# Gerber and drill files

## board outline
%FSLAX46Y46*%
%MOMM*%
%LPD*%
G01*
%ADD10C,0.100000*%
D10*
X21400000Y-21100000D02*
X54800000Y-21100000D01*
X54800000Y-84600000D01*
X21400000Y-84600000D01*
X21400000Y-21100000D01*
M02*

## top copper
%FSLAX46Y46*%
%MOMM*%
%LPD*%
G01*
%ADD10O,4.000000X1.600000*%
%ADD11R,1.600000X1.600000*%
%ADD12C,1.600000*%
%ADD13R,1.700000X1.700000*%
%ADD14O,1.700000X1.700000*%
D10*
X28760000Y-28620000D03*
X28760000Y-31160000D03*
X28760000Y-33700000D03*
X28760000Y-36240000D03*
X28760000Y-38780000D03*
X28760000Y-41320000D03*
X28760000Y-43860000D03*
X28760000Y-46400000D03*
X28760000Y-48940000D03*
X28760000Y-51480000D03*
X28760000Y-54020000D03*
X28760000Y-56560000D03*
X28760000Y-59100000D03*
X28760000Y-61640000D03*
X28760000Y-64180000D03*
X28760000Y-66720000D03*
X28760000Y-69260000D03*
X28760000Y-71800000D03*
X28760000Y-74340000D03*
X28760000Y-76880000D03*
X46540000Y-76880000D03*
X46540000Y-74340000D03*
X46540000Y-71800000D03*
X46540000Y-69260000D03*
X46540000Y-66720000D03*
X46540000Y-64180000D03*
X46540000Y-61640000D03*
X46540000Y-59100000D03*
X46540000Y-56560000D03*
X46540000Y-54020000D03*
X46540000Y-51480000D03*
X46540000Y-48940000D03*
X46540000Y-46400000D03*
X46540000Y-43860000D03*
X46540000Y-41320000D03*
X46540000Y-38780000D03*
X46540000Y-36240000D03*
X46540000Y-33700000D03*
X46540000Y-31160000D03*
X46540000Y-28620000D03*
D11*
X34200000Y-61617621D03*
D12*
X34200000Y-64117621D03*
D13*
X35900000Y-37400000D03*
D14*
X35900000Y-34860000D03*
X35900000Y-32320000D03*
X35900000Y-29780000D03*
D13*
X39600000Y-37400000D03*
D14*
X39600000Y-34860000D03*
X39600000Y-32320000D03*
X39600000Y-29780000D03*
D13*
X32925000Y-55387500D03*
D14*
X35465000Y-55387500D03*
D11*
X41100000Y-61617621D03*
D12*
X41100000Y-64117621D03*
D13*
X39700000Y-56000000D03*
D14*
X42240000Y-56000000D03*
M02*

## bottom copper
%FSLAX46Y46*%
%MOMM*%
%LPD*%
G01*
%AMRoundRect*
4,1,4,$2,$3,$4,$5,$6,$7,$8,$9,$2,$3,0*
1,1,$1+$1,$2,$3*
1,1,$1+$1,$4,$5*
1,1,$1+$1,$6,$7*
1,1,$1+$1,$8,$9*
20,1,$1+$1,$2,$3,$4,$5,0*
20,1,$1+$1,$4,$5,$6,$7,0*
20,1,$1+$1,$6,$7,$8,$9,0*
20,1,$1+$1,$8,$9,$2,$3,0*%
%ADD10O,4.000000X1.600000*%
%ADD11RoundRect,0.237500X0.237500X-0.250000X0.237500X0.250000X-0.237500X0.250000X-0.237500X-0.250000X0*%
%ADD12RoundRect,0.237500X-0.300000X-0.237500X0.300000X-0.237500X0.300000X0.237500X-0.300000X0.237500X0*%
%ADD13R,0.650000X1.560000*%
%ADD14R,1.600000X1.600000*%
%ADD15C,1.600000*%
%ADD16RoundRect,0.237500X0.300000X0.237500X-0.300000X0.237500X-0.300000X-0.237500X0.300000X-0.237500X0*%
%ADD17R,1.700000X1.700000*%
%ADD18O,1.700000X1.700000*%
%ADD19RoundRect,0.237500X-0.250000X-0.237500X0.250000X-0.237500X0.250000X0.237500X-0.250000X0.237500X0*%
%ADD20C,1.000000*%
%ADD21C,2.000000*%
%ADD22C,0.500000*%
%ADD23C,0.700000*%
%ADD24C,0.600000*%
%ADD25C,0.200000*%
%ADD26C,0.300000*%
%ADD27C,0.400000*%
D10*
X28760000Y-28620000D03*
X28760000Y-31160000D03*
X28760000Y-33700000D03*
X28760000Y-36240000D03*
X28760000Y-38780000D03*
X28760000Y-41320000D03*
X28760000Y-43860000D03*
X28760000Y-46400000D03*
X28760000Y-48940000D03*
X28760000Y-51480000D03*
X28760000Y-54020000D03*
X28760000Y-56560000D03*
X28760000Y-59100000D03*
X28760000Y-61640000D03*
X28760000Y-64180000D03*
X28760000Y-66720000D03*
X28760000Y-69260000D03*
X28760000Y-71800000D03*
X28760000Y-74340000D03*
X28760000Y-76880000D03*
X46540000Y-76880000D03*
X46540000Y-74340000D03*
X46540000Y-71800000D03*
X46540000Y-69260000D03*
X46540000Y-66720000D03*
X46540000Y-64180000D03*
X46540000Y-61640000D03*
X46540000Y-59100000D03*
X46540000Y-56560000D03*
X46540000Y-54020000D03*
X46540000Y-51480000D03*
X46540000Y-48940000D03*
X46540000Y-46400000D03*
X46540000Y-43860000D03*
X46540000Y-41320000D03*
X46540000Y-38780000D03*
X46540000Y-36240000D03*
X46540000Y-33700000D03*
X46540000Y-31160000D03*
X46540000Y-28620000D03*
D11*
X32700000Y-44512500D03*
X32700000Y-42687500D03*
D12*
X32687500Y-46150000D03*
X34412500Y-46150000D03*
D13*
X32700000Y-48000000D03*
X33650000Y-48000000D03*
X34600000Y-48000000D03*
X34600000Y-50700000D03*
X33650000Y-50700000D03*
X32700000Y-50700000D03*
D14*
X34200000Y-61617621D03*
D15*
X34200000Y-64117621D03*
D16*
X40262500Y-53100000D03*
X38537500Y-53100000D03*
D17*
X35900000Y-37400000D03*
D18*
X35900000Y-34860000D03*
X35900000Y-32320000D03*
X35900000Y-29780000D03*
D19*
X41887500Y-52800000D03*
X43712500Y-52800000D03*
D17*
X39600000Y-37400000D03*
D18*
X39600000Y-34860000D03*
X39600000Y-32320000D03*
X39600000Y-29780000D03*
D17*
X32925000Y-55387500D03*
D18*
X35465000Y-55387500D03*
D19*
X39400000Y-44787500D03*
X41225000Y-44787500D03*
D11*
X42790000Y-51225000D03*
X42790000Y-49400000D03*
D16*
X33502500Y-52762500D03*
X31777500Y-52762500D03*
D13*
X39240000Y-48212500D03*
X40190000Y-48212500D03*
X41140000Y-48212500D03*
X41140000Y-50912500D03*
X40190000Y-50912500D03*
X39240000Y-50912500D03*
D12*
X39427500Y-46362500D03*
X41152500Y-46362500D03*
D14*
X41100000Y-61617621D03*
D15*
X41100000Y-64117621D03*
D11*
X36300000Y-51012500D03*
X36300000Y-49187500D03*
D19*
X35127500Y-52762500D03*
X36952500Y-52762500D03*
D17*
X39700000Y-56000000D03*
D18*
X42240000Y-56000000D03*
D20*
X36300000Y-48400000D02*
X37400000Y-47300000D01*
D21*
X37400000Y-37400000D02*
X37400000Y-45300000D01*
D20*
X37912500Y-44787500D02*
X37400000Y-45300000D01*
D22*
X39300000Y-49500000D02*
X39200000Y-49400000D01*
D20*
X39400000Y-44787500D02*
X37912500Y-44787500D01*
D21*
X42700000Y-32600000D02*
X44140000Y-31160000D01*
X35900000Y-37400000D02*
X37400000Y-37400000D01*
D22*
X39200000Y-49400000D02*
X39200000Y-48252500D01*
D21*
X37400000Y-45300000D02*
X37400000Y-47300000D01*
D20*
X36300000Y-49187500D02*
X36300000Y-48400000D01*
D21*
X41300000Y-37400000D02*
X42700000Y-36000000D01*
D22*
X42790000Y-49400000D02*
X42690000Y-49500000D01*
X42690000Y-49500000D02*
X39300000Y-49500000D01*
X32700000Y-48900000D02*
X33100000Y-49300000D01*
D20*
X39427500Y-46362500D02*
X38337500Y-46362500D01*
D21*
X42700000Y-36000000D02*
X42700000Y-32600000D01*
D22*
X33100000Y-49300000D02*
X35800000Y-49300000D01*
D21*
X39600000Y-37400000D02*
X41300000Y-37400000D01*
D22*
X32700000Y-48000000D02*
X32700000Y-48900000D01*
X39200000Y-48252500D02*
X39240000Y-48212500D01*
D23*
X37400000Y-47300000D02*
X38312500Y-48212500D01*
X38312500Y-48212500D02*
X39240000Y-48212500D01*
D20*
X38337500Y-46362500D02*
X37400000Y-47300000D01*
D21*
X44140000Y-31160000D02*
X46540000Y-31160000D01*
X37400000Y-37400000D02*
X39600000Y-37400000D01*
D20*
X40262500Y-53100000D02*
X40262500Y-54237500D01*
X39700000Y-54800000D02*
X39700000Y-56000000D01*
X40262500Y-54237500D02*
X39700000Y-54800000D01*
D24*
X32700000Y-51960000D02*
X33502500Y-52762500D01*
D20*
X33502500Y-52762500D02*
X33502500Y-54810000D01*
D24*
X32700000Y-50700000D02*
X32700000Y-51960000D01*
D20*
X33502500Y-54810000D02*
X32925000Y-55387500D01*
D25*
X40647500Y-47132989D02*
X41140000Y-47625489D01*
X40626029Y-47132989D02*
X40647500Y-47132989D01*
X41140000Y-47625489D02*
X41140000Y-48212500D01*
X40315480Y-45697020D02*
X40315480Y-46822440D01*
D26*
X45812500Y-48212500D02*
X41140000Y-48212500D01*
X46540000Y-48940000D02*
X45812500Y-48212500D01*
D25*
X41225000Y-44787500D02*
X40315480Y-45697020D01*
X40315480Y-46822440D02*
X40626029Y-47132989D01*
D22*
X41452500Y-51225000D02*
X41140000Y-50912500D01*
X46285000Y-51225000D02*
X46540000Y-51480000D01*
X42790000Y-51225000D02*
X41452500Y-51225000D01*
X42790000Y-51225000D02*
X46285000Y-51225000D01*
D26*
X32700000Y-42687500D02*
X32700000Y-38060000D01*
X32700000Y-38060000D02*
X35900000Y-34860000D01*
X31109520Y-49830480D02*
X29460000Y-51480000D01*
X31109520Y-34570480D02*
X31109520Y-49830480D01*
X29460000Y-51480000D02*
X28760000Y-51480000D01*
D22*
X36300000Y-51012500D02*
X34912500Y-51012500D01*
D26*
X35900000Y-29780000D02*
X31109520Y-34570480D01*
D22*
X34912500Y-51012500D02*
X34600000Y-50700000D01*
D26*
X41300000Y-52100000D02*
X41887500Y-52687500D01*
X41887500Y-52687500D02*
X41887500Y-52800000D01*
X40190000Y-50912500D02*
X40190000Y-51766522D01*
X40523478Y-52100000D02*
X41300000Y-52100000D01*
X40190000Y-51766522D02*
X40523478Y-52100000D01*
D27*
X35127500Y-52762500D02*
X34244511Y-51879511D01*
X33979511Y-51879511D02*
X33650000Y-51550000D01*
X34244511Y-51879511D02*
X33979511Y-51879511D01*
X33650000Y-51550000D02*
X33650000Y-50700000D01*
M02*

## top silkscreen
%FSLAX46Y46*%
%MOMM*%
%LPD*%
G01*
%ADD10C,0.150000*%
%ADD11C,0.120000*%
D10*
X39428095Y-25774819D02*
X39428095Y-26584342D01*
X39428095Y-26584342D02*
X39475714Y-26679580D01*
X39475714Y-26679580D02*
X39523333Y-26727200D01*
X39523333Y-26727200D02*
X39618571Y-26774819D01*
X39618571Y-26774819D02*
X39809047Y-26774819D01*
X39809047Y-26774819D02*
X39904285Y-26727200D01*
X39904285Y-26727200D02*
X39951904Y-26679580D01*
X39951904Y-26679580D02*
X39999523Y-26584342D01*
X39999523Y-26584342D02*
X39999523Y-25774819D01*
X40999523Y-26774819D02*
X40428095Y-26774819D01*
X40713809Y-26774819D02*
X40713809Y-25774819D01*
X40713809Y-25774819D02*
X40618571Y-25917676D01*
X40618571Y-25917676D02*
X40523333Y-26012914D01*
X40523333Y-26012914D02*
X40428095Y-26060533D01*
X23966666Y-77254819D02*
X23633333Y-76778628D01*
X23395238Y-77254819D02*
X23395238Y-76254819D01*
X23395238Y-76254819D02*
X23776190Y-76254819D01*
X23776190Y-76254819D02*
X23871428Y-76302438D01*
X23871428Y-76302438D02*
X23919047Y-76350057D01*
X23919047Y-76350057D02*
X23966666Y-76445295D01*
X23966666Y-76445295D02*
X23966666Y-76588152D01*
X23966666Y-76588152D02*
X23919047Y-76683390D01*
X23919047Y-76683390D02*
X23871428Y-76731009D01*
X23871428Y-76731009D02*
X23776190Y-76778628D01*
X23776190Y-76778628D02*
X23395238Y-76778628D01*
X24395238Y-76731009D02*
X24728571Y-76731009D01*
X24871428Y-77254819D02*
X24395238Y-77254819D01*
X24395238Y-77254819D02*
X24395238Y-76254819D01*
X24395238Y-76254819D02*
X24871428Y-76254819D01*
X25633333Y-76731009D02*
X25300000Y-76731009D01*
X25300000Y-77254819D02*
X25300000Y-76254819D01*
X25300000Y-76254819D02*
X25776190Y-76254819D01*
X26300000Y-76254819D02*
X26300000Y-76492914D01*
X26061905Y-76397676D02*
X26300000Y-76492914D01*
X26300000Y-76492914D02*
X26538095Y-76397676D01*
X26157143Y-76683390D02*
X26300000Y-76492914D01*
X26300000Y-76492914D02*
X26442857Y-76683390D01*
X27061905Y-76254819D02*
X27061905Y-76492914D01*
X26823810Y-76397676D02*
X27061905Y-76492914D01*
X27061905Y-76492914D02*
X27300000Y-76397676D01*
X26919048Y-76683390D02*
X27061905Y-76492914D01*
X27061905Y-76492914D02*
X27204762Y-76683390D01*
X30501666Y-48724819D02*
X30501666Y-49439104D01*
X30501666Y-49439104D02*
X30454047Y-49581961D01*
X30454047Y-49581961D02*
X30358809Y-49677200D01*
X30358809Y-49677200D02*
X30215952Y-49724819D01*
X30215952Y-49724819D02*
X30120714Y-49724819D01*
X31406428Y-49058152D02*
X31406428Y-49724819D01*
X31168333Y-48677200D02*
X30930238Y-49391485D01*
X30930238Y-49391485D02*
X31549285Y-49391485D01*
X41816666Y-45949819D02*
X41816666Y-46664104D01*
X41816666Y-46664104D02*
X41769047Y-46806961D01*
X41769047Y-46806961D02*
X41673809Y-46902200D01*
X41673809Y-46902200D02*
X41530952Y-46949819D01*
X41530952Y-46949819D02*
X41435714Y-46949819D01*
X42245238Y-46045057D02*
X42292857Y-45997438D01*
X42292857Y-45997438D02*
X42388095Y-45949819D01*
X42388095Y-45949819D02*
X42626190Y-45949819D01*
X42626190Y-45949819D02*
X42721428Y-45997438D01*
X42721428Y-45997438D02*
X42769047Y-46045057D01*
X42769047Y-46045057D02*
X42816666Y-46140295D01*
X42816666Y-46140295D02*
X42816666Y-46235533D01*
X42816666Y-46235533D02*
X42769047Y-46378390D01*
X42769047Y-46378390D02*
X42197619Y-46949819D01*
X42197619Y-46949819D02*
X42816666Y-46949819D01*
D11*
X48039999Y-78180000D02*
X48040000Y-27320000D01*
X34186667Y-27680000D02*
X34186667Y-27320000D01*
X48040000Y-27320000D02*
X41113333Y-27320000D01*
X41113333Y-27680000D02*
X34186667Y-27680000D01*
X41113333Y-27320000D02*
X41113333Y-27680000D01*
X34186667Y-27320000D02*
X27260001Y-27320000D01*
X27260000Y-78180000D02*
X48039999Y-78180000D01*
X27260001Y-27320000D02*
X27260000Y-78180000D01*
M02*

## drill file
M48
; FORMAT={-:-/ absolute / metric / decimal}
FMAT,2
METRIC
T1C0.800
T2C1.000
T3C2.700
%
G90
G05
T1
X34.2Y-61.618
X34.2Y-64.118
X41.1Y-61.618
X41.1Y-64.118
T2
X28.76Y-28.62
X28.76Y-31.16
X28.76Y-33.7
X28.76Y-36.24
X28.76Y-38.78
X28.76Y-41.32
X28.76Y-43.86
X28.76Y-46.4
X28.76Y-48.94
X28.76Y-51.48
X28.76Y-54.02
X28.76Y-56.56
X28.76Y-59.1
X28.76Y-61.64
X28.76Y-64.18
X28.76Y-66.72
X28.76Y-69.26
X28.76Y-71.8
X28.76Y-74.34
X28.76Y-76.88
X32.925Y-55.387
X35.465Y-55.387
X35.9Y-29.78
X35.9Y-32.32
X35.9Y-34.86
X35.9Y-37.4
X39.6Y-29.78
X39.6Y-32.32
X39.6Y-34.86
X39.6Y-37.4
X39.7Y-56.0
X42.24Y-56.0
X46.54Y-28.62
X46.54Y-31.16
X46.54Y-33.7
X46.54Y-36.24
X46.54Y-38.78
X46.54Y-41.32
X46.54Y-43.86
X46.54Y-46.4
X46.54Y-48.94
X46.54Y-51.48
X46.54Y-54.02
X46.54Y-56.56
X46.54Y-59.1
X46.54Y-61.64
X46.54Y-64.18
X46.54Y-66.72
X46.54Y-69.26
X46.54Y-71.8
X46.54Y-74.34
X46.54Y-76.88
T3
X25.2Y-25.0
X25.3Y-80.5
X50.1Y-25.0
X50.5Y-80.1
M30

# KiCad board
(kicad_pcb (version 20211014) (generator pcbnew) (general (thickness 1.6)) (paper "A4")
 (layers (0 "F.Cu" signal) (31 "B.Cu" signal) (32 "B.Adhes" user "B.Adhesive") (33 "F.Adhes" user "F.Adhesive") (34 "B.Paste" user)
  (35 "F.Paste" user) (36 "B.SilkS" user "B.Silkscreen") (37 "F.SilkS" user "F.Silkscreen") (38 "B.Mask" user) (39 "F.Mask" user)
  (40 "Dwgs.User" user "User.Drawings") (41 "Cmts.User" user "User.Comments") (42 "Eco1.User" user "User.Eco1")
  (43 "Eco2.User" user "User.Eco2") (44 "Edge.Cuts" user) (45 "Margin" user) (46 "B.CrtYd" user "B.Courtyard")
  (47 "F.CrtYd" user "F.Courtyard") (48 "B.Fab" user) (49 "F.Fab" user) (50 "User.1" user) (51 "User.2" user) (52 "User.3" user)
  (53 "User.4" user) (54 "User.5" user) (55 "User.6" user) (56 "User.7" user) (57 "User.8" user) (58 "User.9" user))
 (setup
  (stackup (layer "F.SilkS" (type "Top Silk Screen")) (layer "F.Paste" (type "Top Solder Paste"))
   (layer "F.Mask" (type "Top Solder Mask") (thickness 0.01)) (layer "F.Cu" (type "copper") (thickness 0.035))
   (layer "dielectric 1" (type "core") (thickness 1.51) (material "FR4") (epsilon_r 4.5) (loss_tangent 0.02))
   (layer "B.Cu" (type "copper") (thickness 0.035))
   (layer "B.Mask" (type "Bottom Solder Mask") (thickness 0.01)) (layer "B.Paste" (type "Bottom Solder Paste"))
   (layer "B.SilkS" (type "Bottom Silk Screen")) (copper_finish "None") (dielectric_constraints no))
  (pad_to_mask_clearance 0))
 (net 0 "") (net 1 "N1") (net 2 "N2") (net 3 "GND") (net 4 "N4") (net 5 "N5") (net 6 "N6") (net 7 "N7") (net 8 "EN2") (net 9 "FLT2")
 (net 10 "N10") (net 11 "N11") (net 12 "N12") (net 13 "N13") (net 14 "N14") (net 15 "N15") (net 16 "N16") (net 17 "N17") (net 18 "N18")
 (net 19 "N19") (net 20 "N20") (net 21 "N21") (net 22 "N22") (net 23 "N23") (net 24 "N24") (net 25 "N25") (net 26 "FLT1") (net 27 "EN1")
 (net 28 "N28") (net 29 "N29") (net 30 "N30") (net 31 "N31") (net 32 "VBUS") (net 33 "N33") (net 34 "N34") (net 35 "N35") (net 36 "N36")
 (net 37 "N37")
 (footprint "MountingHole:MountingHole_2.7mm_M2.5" (layer "F.Cu") (at 50.5 80.1)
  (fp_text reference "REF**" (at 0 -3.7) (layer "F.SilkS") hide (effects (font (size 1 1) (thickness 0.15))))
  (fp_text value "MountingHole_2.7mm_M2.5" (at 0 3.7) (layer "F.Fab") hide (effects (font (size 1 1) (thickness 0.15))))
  (pad "" np_thru_hole circle (at 0 0) (size 2.7 2.7) (drill 2.7) (layers *.Cu *.Mask)))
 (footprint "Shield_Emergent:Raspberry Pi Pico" (layer "F.Cu") (at 37.65 52.75 -90)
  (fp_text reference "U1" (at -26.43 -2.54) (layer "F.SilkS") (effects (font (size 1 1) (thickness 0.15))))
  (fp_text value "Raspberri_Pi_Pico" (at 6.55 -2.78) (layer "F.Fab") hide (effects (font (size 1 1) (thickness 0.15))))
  (fp_line (start 25.43 -10.389999) (end -25.43 -10.39) (layer "F.SilkS") (width 0.12))
  (fp_line (start -25.07 3.463333) (end -25.43 3.463333) (layer "F.SilkS") (width 0.12))
  (fp_line (start -25.43 -10.39) (end -25.43 -3.463333) (layer "F.SilkS") (width 0.12))
  (fp_line (start -25.07 -3.463333) (end -25.07 3.463333) (layer "F.SilkS") (width 0.12))
  (fp_line (start -25.43 -3.463333) (end -25.07 -3.463333) (layer "F.SilkS") (width 0.12))
  (fp_line (start -25.43 3.463333) (end -25.43 10.389999) (layer "F.SilkS") (width 0.12))
  (fp_line (start 25.43 10.39) (end 25.43 -10.389999) (layer "F.SilkS") (width 0.12))
  (fp_line (start -25.43 10.389999) (end 25.43 10.39) (layer "F.SilkS") (width 0.12))
  (pad "1" thru_hole oval (at -24.13 8.89 270) (size 1.6 4) (drill 1) (layers *.Cu *.Mask) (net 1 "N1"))
  (pad "2" thru_hole oval (at -21.59 8.89 270) (size 1.6 4) (drill 1) (layers *.Cu *.Mask) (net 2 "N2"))
  (pad "3" thru_hole oval (at -19.05 8.89 270) (size 1.6 4) (drill 1) (layers *.Cu *.Mask) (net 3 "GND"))
  (pad "4" thru_hole oval (at -16.51 8.89 270) (size 1.6 4) (drill 1) (layers *.Cu *.Mask) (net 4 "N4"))
  (pad "5" thru_hole oval (at -13.97 8.89 270) (size 1.6 4) (drill 1) (layers *.Cu *.Mask) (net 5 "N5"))
  (pad "6" thru_hole oval (at -11.43 8.89 270) (size 1.6 4) (drill 1) (layers *.Cu *.Mask) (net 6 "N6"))
  (pad "7" thru_hole oval (at -8.89 8.89 270) (size 1.6 4) (drill 1) (layers *.Cu *.Mask) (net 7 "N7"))
  (pad "8" thru_hole oval (at -6.35 8.89 270) (size 1.6 4) (drill 1) (layers *.Cu *.Mask) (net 3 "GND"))
  (pad "9" thru_hole oval (at -3.81 8.89 270) (size 1.6 4) (drill 1) (layers *.Cu *.Mask) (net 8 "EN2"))
  (pad "10" thru_hole oval (at -1.27 8.89 270) (size 1.6 4) (drill 1) (layers *.Cu *.Mask) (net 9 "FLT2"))
  (pad "11" thru_hole oval (at 1.27 8.89 270) (size 1.6 4) (drill 1) (layers *.Cu *.Mask) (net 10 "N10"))
  (pad "12" thru_hole oval (at 3.81 8.89 270) (size 1.6 4) (drill 1) (layers *.Cu *.Mask) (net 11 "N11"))
  (pad "13" thru_hole oval (at 6.35 8.89 270) (size 1.6 4) (drill 1) (layers *.Cu *.Mask) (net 3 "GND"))
  (pad "14" thru_hole oval (at 8.89 8.89 270) (size 1.6 4) (drill 1) (layers *.Cu *.Mask) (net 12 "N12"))
  (pad "15" thru_hole oval (at 11.43 8.89 270) (size 1.6 4) (drill 1) (layers *.Cu *.Mask) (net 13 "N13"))
  (pad "16" thru_hole oval (at 13.97 8.89 270) (size 1.6 4) (drill 1) (layers *.Cu *.Mask) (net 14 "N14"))
  (pad "17" thru_hole oval (at 16.51 8.89 270) (size 1.6 4) (drill 1) (layers *.Cu *.Mask) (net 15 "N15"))
  (pad "18" thru_hole oval (at 19.05 8.89 270) (size 1.6 4) (drill 1) (layers *.Cu *.Mask) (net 3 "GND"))
  (pad "19" thru_hole oval (at 21.59 8.89 270) (size 1.6 4) (drill 1) (layers *.Cu *.Mask) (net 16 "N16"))
  (pad "20" thru_hole oval (at 24.13 8.89 270) (size 1.6 4) (drill 1) (layers *.Cu *.Mask) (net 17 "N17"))
  (pad "21" thru_hole oval (at 24.13 -8.89 270) (size 1.6 4) (drill 1) (layers *.Cu *.Mask) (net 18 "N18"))
  (pad "22" thru_hole oval (at 21.59 -8.89 270) (size 1.6 4) (drill 1) (layers *.Cu *.Mask) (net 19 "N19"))
  (pad "23" thru_hole oval (at 19.05 -8.89 270) (size 1.6 4) (drill 1) (layers *.Cu *.Mask) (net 3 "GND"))
  (pad "24" thru_hole oval (at 16.51 -8.89 270) (size 1.6 4) (drill 1) (layers *.Cu *.Mask) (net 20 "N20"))
  (pad "25" thru_hole oval (at 13.97 -8.89 270) (size 1.6 4) (drill 1) (layers *.Cu *.Mask) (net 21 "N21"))
  (pad "26" thru_hole oval (at 11.43 -8.89 270) (size 1.6 4) (drill 1) (layers *.Cu *.Mask) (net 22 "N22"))
  (pad "27" thru_hole oval (at 8.89 -8.89 270) (size 1.6 4) (drill 1) (layers *.Cu *.Mask) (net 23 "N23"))
  (pad "28" thru_hole oval (at 6.35 -8.89 270) (size 1.6 4) (drill 1) (layers *.Cu *.Mask) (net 3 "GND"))
  (pad "29" thru_hole oval (at 3.81 -8.89 270) (size 1.6 4) (drill 1) (layers *.Cu *.Mask) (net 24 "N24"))
  (pad "30" thru_hole oval (at 1.27 -8.89 270) (size 1.6 4) (drill 1) (layers *.Cu *.Mask) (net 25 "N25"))
  (pad "31" thru_hole oval (at -1.27 -8.89 270) (size 1.6 4) (drill 1) (layers *.Cu *.Mask) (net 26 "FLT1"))
  (pad "32" thru_hole oval (at -3.81 -8.89 270) (size 1.6 4) (drill 1) (layers *.Cu *.Mask) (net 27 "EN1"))
  (pad "33" thru_hole oval (at -6.35 -8.89 270) (size 1.6 4) (drill 1) (layers *.Cu *.Mask) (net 3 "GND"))
  (pad "34" thru_hole oval (at -8.89 -8.89 270) (size 1.6 4) (drill 1) (layers *.Cu *.Mask) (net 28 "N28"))
  (pad "35" thru_hole oval (at -11.43 -8.89 270) (size 1.6 4) (drill 1) (layers *.Cu *.Mask) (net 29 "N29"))
  (pad "36" thru_hole oval (at -13.97 -8.89 270) (size 1.6 4) (drill 1) (layers *.Cu *.Mask) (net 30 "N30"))
  (pad "37" thru_hole oval (at -16.51 -8.89 270) (size 1.6 4) (drill 1) (layers *.Cu *.Mask) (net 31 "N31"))
  (pad "38" thru_hole oval (at -19.05 -8.89 270) (size 1.6 4) (drill 1) (layers *.Cu *.Mask) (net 3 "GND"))
  (pad "39" thru_hole oval (at -21.59 -8.89 270) (size 1.6 4) (drill 1) (layers *.Cu *.Mask) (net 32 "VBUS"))
  (pad "40" thru_hole oval (at -24.13 -8.89 270) (size 1.6 4) (drill 1) (layers *.Cu *.Mask) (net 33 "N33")))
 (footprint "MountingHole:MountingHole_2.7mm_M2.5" (layer "F.Cu") (at 25.3 80.5)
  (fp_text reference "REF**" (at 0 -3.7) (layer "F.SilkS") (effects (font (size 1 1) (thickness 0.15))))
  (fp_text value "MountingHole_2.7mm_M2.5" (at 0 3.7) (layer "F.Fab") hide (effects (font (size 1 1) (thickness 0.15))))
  (pad "" np_thru_hole circle (at 0 0) (size 2.7 2.7) (drill 2.7) (layers *.Cu *.Mask)))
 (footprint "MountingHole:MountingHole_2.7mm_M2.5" (layer "F.Cu") (at 25.2 25)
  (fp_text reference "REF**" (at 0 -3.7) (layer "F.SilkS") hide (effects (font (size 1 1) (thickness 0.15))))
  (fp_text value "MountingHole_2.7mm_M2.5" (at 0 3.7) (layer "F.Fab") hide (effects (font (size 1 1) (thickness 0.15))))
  (pad "" np_thru_hole circle (at 0 0) (size 2.7 2.7) (drill 2.7) (layers *.Cu *.Mask)))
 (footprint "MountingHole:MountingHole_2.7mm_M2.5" (layer "F.Cu") (at 50.1 25)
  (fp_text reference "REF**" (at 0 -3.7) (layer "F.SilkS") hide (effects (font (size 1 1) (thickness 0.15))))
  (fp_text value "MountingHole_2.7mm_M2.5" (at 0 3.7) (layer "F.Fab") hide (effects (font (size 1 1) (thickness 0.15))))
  (pad "" np_thru_hole circle (at 0 0) (size 2.7 2.7) (drill 2.7) (layers *.Cu *.Mask)))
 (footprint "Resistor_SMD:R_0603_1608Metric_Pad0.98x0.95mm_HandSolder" (layer "B.Cu") (at 32.7 43.6 90)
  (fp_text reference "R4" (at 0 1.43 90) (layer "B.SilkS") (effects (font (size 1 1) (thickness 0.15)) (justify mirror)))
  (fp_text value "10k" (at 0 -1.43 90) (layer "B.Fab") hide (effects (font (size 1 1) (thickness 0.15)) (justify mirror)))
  (pad "1" smd roundrect (at -0.9125 0 90) (size 0.975 0.95) (layers "B.Cu" "B.Paste" "B.Mask") (roundrect_rratio 0.25) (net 32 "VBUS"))
  (pad "2" smd roundrect (at 0.9125 0 90) (size 0.975 0.95) (layers "B.Cu" "B.Paste" "B.Mask") (roundrect_rratio 0.25) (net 8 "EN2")))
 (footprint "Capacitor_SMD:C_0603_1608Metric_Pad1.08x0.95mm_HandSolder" (layer "B.Cu") (at 33.55 46.15)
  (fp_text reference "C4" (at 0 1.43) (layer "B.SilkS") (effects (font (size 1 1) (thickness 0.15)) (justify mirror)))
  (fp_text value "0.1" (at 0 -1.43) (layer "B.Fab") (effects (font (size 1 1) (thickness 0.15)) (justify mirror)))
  (pad "1" smd roundrect (at -0.8625 0) (size 1.075 0.95) (layers "B.Cu" "B.Paste" "B.Mask") (roundrect_rratio 0.25) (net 32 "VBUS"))
  (pad "2" smd roundrect (at 0.8625 0) (size 1.075 0.95) (layers "B.Cu" "B.Paste" "B.Mask") (roundrect_rratio 0.25) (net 3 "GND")))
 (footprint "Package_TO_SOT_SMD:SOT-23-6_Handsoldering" (layer "B.Cu") (at 33.65 49.35 -90)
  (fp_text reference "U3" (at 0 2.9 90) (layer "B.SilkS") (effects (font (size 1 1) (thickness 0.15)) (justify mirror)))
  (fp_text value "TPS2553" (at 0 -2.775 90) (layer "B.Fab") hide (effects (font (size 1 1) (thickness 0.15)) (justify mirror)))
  (pad "1" smd rect (at -1.35 0.95 270) (size 1.56 0.65) (layers "B.Cu" "B.Paste" "B.Mask") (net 32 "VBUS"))
  (pad "2" smd rect (at -1.35 0 270) (size 1.56 0.65) (layers "B.Cu" "B.Paste" "B.Mask") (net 3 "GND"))
  (pad "3" smd rect (at -1.35 -0.95 270) (size 1.56 0.65) (layers "B.Cu" "B.Paste" "B.Mask") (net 8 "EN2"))
  (pad "4" smd rect (at 1.35 -0.95 270) (size 1.56 0.65) (layers "B.Cu" "B.Paste" "B.Mask") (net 9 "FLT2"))
  (pad "5" smd rect (at 1.35 0 270) (size 1.56 0.65) (layers "B.Cu" "B.Paste" "B.Mask") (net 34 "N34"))
  (pad "6" smd rect (at 1.35 0.95 270) (size 1.56 0.65) (layers "B.Cu" "B.Paste" "B.Mask") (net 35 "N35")))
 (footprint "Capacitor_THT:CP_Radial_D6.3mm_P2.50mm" (layer "B.Cu") (at 34.2 61.617621 -90)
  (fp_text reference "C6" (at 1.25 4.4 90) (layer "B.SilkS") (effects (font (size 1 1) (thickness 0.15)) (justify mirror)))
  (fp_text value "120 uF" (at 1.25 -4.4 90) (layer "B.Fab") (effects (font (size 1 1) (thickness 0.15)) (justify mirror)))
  (pad "1" thru_hole rect (at 0 0 270) (size 1.6 1.6) (drill 0.8) (layers *.Cu *.Mask) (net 35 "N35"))
  (pad "2" thru_hole circle (at 2.5 0 270) (size 1.6 1.6) (drill 0.8) (layers *.Cu *.Mask) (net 3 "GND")))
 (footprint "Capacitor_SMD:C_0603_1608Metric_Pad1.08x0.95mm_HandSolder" (layer "B.Cu") (at 39.4 53.1 180)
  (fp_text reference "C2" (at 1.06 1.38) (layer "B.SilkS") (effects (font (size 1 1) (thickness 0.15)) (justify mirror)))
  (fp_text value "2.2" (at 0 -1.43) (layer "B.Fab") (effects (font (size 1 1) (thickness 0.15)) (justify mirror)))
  (pad "1" smd roundrect (at -0.8625 0 180) (size 1.075 0.95) (layers "B.Cu" "B.Paste" "B.Mask") (roundrect_rratio 0.25) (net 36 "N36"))
  (pad "2" smd roundrect (at 0.8625 0 180) (size 1.075 0.95) (layers "B.Cu" "B.Paste" "B.Mask") (roundrect_rratio 0.25) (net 3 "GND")))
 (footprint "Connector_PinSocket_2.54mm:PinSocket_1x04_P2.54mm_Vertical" (layer "B.Cu") (at 35.9 37.4)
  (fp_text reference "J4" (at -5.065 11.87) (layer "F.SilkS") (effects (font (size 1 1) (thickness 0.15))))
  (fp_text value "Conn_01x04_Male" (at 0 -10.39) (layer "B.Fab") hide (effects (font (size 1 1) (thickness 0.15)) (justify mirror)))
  (pad "1" thru_hole rect (at 0 0) (size 1.7 1.7) (drill 1) (layers *.Cu *.Mask) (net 32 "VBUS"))
  (pad "2" thru_hole oval (at 0 -2.54) (size 1.7 1.7) (drill 1) (layers *.Cu *.Mask) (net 8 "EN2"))
  (pad "3" thru_hole oval (at 0 -5.08) (size 1.7 1.7) (drill 1) (layers *.Cu *.Mask) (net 3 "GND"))
  (pad "4" thru_hole oval (at 0 -7.62) (size 1.7 1.7) (drill 1) (layers *.Cu *.Mask) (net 9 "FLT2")))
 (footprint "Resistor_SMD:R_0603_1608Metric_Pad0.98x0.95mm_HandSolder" (layer "B.Cu") (at 42.8 52.8)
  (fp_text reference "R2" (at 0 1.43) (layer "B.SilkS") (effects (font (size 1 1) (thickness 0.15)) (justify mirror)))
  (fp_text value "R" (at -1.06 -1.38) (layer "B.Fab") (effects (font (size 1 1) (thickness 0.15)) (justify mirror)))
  (pad "1" smd roundrect (at -0.9125 0) (size 0.975 0.95) (layers "B.Cu" "B.Paste" "B.Mask") (roundrect_rratio 0.25) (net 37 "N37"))
  (pad "2" smd roundrect (at 0.9125 0) (size 0.975 0.95) (layers "B.Cu" "B.Paste" "B.Mask") (roundrect_rratio 0.25) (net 3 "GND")))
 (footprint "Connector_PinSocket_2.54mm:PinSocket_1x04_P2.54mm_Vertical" (layer "B.Cu") (at 39.6 37.4)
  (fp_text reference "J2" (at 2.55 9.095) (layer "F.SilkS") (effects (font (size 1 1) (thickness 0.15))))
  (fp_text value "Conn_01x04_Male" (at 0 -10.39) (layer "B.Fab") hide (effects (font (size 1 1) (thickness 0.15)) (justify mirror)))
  (pad "1" thru_hole rect (at 0 0) (size 1.7 1.7) (drill 1) (layers *.Cu *.Mask) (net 32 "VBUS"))
  (pad "2" thru_hole oval (at 0 -2.54) (size 1.7 1.7) (drill 1) (layers *.Cu *.Mask) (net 27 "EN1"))
  (pad "3" thru_hole oval (at 0 -5.08) (size 1.7 1.7) (drill 1) (layers *.Cu *.Mask) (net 3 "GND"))
  (pad "4" thru_hole oval (at 0 -7.62) (size 1.7 1.7) (drill 1) (layers *.Cu *.Mask) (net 26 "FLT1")))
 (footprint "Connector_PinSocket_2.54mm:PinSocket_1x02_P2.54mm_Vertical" (layer "B.Cu") (at 32.925 55.3875 -90)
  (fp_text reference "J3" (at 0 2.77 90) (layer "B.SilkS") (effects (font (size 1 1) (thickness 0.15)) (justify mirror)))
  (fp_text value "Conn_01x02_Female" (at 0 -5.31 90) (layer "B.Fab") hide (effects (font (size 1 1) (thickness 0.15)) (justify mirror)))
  (pad "1" thru_hole rect (at 0 0 270) (size 1.7 1.7) (drill 1) (layers *.Cu *.Mask) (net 35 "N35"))
  (pad "2" thru_hole oval (at 0 -2.54 270) (size 1.7 1.7) (drill 1) (layers *.Cu *.Mask) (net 3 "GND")))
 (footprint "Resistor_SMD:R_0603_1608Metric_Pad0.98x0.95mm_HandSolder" (layer "B.Cu") (at 40.3125 44.7875)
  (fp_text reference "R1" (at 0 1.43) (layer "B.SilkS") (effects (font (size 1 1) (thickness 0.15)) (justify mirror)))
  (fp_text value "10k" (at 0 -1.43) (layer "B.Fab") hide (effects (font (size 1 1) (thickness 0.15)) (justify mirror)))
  (pad "1" smd roundrect (at -0.9125 0) (size 0.975 0.95) (layers "B.Cu" "B.Paste" "B.Mask") (roundrect_rratio 0.25) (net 32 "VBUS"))
  (pad "2" smd roundrect (at 0.9125 0) (size 0.975 0.95) (layers "B.Cu" "B.Paste" "B.Mask") (roundrect_rratio 0.25) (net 27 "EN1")))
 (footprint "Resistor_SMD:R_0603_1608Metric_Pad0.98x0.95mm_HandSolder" (layer "B.Cu") (at 42.79 50.3125 90)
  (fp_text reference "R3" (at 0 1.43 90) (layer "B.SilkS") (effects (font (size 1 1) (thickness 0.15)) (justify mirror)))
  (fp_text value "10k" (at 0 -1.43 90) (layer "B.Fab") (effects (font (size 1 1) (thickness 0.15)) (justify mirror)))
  (pad "1" smd roundrect (at -0.9125 0 90) (size 0.975 0.95) (layers "B.Cu" "B.Paste" "B.Mask") (roundrect_rratio 0.25) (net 26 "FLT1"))
  (pad "2" smd roundrect (at 0.9125 0 90) (size 0.975 0.95) (layers "B.Cu" "B.Paste" "B.Mask") (roundrect_rratio 0.25) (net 32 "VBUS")))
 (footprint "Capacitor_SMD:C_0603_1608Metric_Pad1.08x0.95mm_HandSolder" (layer "B.Cu") (at 32.64 52.7625 180)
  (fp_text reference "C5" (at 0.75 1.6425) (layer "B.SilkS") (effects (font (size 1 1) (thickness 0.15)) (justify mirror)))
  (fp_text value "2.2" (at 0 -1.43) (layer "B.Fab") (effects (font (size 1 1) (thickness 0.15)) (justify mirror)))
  (pad "1" smd roundrect (at -0.8625 0 180) (size 1.075 0.95) (layers "B.Cu" "B.Paste" "B.Mask") (roundrect_rratio 0.25) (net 35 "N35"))
  (pad "2" smd roundrect (at 0.8625 0 180) (size 1.075 0.95) (layers "B.Cu" "B.Paste" "B.Mask") (roundrect_rratio 0.25) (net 3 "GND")))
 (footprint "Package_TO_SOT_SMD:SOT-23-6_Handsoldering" (layer "B.Cu") (at 40.19 49.5625 -90)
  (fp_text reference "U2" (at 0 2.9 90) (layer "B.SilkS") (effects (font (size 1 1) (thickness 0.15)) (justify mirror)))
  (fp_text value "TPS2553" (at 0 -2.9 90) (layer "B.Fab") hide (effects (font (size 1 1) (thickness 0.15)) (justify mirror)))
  (pad "1" smd rect (at -1.35 0.95 270) (size 1.56 0.65) (layers "B.Cu" "B.Paste" "B.Mask") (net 32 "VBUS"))
  (pad "2" smd rect (at -1.35 0 270) (size 1.56 0.65) (layers "B.Cu" "B.Paste" "B.Mask") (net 3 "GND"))
  (pad "3" smd rect (at -1.35 -0.95 270) (size 1.56 0.65) (layers "B.Cu" "B.Paste" "B.Mask") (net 27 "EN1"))
  (pad "4" smd rect (at 1.35 -0.95 270) (size 1.56 0.65) (layers "B.Cu" "B.Paste" "B.Mask") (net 26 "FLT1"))
  (pad "5" smd rect (at 1.35 0 270) (size 1.56 0.65) (layers "B.Cu" "B.Paste" "B.Mask") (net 37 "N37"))
  (pad "6" smd rect (at 1.35 0.95 270) (size 1.56 0.65) (layers "B.Cu" "B.Paste" "B.Mask") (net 36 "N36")))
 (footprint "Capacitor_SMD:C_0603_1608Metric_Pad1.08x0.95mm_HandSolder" (layer "B.Cu") (at 40.29 46.3625)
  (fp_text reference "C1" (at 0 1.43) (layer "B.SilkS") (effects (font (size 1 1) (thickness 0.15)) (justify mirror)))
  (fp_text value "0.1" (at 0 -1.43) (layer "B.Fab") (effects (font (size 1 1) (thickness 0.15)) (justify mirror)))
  (pad "1" smd roundrect (at -0.8625 0) (size 1.075 0.95) (layers "B.Cu" "B.Paste" "B.Mask") (roundrect_rratio 0.25) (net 32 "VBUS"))
  (pad "2" smd roundrect (at 0.8625 0) (size 1.075 0.95) (layers "B.Cu" "B.Paste" "B.Mask") (roundrect_rratio 0.25) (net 3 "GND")))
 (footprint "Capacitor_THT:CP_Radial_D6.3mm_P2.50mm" (layer "B.Cu") (at 41.1 61.617621 -90)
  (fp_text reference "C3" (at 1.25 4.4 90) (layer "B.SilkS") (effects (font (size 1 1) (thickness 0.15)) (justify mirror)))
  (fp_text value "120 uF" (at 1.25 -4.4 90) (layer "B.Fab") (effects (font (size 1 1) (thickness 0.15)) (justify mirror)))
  (pad "1" thru_hole rect (at 0 0 270) (size 1.6 1.6) (drill 0.8) (layers *.Cu *.Mask) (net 36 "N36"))
  (pad "2" thru_hole circle (at 2.5 0 270) (size 1.6 1.6) (drill 0.8) (layers *.Cu *.Mask) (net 3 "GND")))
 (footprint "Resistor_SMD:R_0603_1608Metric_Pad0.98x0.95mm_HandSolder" (layer "B.Cu") (at 36.3 50.1 90)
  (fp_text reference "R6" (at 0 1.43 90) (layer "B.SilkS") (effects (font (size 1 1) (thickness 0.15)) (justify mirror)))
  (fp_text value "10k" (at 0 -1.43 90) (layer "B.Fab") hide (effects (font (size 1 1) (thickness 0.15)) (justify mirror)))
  (pad "1" smd roundrect (at -0.9125 0 90) (size 0.975 0.95) (layers "B.Cu" "B.Paste" "B.Mask") (roundrect_rratio 0.25) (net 9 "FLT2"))
  (pad "2" smd roundrect (at 0.9125 0 90) (size 0.975 0.95) (layers "B.Cu" "B.Paste" "B.Mask") (roundrect_rratio 0.25) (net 32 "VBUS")))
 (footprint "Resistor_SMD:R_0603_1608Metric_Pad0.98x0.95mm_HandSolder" (layer "B.Cu") (at 36.04 52.7625)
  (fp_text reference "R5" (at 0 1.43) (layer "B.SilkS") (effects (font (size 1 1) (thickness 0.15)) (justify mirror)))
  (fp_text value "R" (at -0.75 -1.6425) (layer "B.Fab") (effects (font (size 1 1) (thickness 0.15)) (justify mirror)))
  (pad "1" smd roundrect (at -0.9125 0) (size 0.975 0.95) (layers "B.Cu" "B.Paste" "B.Mask") (roundrect_rratio 0.25) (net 34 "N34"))
  (pad "2" smd roundrect (at 0.9125 0) (size 0.975 0.95) (layers "B.Cu" "B.Paste" "B.Mask") (roundrect_rratio 0.25) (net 3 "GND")))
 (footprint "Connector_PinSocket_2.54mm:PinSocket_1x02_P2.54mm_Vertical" (layer "B.Cu") (at 39.7 56 -90)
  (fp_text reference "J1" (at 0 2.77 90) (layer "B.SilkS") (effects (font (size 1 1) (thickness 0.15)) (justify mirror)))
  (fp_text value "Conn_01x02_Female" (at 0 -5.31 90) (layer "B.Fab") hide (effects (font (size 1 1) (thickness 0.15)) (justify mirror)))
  (pad "1" thru_hole rect (at 0 0 270) (size 1.7 1.7) (drill 1) (layers *.Cu *.Mask) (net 36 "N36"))
  (pad "2" thru_hole oval (at 0 -2.54 270) (size 1.7 1.7) (drill 1) (layers *.Cu *.Mask) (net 3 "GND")))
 (gr_rect (start 21.4 21.1) (end 54.8 84.6) (layer "Edge.Cuts") (width 0.1) (fill none))
 (segment (start 36.3 48.4) (end 37.4 47.3) (width 1) (layer "B.Cu") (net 32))
 (segment (start 37.4 37.4) (end 37.4 45.3) (width 2) (layer "B.Cu") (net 32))
 (segment (start 37.9125 44.7875) (end 37.4 45.3) (width 1) (layer "B.Cu") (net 32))
 (segment (start 39.3 49.5) (end 39.2 49.4) (width 0.5) (layer "B.Cu") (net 32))
 (segment (start 39.4 44.7875) (end 37.9125 44.7875) (width 1) (layer "B.Cu") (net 32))
 (segment (start 42.7 32.6) (end 44.14 31.16) (width 2) (layer "B.Cu") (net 32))
 (segment (start 35.9 37.4) (end 37.4 37.4) (width 2) (layer "B.Cu") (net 32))
 (segment (start 39.2 49.4) (end 39.2 48.2525) (width 0.5) (layer "B.Cu") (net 32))
 (segment (start 37.4 45.3) (end 37.4 47.3) (width 2) (layer "B.Cu") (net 32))
 (segment (start 36.3 49.1875) (end 36.3 48.4) (width 1) (layer "B.Cu") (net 32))
 (segment (start 41.3 37.4) (end 42.7 36) (width 2) (layer "B.Cu") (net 32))
 (segment (start 42.79 49.4) (end 42.69 49.5) (width 0.5) (layer "B.Cu") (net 32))
 (segment (start 42.69 49.5) (end 39.3 49.5) (width 0.5) (layer "B.Cu") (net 32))
 (segment (start 32.7 48.9) (end 33.1 49.3) (width 0.5) (layer "B.Cu") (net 32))
 (segment (start 39.4275 46.3625) (end 38.3375 46.3625) (width 1) (layer "B.Cu") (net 32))
 (segment (start 42.7 36) (end 42.7 32.6) (width 2) (layer "B.Cu") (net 32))
 (segment (start 33.1 49.3) (end 35.8 49.3) (width 0.5) (layer "B.Cu") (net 32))
 (segment (start 39.6 37.4) (end 41.3 37.4) (width 2) (layer "B.Cu") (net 32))
 (segment (start 32.7 48) (end 32.7 48.9) (width 0.5) (layer "B.Cu") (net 32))
 (segment (start 39.2 48.2525) (end 39.24 48.2125) (width 0.5) (layer "B.Cu") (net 32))
 (segment (start 37.4 47.3) (end 38.3125 48.2125) (width 0.7) (layer "B.Cu") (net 32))
 (segment (start 38.3125 48.2125) (end 39.24 48.2125) (width 0.7) (layer "B.Cu") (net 32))
 (segment (start 38.3375 46.3625) (end 37.4 47.3) (width 1) (layer "B.Cu") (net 32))
 (segment (start 44.14 31.16) (end 46.54 31.16) (width 2) (layer "B.Cu") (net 32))
 (segment (start 37.4 37.4) (end 39.6 37.4) (width 2) (layer "B.Cu") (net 32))
 (segment (start 40.2625 53.1) (end 40.2625 54.2375) (width 1) (layer "B.Cu") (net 36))
 (segment (start 39.7 54.8) (end 39.7 56) (width 1) (layer "B.Cu") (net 36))
 (segment (start 40.2625 54.2375) (end 39.7 54.8) (width 1) (layer "B.Cu") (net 36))
 (segment (start 32.7 51.96) (end 33.5025 52.7625) (width 0.6) (layer "B.Cu") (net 35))
 (segment (start 33.5025 52.7625) (end 33.5025 54.81) (width 1) (layer "B.Cu") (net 35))
 (segment (start 32.7 50.7) (end 32.7 51.96) (width 0.6) (layer "B.Cu") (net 35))
 (segment (start 33.5025 54.81) (end 32.925 55.3875) (width 1) (layer "B.Cu") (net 35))
 (segment (start 40.6475 47.132989) (end 41.14 47.625489) (width 0.2) (layer "B.Cu") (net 27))
 (segment (start 40.626029 47.132989) (end 40.6475 47.132989) (width 0.2) (layer "B.Cu") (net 27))
 (segment (start 41.14 47.625489) (end 41.14 48.2125) (width 0.2) (layer "B.Cu") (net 27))
 (segment (start 40.31548 45.69702) (end 40.31548 46.82244) (width 0.2) (layer "B.Cu") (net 27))
 (segment (start 45.8125 48.2125) (end 41.14 48.2125) (width 0.3) (layer "B.Cu") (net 27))
 (segment (start 46.54 48.94) (end 45.8125 48.2125) (width 0.3) (layer "B.Cu") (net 27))
 (segment (start 41.225 44.7875) (end 40.31548 45.69702) (width 0.2) (layer "B.Cu") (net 27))
 (segment (start 40.31548 46.82244) (end 40.626029 47.132989) (width 0.2) (layer "B.Cu") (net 27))
 (segment (start 41.4525 51.225) (end 41.14 50.9125) (width 0.5) (layer "B.Cu") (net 26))
 (segment (start 46.285 51.225) (end 46.54 51.48) (width 0.5) (layer "B.Cu") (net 26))
 (segment (start 42.79 51.225) (end 41.4525 51.225) (width 0.5) (layer "B.Cu") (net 26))
 (segment (start 42.79 51.225) (end 46.285 51.225) (width 0.5) (layer "B.Cu") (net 26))
 (segment (start 32.7 42.6875) (end 32.7 38.06) (width 0.3) (layer "B.Cu") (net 8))
 (segment (start 32.7 38.06) (end 35.9 34.86) (width 0.3) (layer "B.Cu") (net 8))
 (segment (start 31.10952 49.83048) (end 29.46 51.48) (width 0.3) (layer "B.Cu") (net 9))
 (segment (start 31.10952 34.57048) (end 31.10952 49.83048) (width 0.3) (layer "B.Cu") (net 9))
 (segment (start 29.46 51.48) (end 28.76 51.48) (width 0.3) (layer "B.Cu") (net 9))
 (segment (start 36.3 51.0125) (end 34.9125 51.0125) (width 0.5) (layer "B.Cu") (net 9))
 (segment (start 35.9 29.78) (end 31.10952 34.57048) (width 0.3) (layer "B.Cu") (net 9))
 (segment (start 34.9125 51.0125) (end 34.6 50.7) (width 0.5) (layer "B.Cu") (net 9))
 (segment (start 41.3 52.1) (end 41.8875 52.6875) (width 0.3) (layer "B.Cu") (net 37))
 (segment (start 41.8875 52.6875) (end 41.8875 52.8) (width 0.3) (layer "B.Cu") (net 37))
 (segment (start 40.19 50.9125) (end 40.19 51.766522) (width 0.3) (layer "B.Cu") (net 37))
 (segment (start 40.523478 52.1) (end 41.3 52.1) (width 0.3) (layer "B.Cu") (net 37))
 (segment (start 40.19 51.766522) (end 40.523478 52.1) (width 0.3) (layer "B.Cu") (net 37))
 (segment (start 35.1275 52.7625) (end 34.244511 51.879511) (width 0.4) (layer "B.Cu") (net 34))
 (segment (start 33.979511 51.879511) (end 33.65 51.55) (width 0.4) (layer "B.Cu") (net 34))
 (segment (start 34.244511 51.879511) (end 33.979511 51.879511) (width 0.4) (layer "B.Cu") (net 34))
 (segment (start 33.65 51.55) (end 33.65 50.7) (width 0.4) (layer "B.Cu") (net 34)))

